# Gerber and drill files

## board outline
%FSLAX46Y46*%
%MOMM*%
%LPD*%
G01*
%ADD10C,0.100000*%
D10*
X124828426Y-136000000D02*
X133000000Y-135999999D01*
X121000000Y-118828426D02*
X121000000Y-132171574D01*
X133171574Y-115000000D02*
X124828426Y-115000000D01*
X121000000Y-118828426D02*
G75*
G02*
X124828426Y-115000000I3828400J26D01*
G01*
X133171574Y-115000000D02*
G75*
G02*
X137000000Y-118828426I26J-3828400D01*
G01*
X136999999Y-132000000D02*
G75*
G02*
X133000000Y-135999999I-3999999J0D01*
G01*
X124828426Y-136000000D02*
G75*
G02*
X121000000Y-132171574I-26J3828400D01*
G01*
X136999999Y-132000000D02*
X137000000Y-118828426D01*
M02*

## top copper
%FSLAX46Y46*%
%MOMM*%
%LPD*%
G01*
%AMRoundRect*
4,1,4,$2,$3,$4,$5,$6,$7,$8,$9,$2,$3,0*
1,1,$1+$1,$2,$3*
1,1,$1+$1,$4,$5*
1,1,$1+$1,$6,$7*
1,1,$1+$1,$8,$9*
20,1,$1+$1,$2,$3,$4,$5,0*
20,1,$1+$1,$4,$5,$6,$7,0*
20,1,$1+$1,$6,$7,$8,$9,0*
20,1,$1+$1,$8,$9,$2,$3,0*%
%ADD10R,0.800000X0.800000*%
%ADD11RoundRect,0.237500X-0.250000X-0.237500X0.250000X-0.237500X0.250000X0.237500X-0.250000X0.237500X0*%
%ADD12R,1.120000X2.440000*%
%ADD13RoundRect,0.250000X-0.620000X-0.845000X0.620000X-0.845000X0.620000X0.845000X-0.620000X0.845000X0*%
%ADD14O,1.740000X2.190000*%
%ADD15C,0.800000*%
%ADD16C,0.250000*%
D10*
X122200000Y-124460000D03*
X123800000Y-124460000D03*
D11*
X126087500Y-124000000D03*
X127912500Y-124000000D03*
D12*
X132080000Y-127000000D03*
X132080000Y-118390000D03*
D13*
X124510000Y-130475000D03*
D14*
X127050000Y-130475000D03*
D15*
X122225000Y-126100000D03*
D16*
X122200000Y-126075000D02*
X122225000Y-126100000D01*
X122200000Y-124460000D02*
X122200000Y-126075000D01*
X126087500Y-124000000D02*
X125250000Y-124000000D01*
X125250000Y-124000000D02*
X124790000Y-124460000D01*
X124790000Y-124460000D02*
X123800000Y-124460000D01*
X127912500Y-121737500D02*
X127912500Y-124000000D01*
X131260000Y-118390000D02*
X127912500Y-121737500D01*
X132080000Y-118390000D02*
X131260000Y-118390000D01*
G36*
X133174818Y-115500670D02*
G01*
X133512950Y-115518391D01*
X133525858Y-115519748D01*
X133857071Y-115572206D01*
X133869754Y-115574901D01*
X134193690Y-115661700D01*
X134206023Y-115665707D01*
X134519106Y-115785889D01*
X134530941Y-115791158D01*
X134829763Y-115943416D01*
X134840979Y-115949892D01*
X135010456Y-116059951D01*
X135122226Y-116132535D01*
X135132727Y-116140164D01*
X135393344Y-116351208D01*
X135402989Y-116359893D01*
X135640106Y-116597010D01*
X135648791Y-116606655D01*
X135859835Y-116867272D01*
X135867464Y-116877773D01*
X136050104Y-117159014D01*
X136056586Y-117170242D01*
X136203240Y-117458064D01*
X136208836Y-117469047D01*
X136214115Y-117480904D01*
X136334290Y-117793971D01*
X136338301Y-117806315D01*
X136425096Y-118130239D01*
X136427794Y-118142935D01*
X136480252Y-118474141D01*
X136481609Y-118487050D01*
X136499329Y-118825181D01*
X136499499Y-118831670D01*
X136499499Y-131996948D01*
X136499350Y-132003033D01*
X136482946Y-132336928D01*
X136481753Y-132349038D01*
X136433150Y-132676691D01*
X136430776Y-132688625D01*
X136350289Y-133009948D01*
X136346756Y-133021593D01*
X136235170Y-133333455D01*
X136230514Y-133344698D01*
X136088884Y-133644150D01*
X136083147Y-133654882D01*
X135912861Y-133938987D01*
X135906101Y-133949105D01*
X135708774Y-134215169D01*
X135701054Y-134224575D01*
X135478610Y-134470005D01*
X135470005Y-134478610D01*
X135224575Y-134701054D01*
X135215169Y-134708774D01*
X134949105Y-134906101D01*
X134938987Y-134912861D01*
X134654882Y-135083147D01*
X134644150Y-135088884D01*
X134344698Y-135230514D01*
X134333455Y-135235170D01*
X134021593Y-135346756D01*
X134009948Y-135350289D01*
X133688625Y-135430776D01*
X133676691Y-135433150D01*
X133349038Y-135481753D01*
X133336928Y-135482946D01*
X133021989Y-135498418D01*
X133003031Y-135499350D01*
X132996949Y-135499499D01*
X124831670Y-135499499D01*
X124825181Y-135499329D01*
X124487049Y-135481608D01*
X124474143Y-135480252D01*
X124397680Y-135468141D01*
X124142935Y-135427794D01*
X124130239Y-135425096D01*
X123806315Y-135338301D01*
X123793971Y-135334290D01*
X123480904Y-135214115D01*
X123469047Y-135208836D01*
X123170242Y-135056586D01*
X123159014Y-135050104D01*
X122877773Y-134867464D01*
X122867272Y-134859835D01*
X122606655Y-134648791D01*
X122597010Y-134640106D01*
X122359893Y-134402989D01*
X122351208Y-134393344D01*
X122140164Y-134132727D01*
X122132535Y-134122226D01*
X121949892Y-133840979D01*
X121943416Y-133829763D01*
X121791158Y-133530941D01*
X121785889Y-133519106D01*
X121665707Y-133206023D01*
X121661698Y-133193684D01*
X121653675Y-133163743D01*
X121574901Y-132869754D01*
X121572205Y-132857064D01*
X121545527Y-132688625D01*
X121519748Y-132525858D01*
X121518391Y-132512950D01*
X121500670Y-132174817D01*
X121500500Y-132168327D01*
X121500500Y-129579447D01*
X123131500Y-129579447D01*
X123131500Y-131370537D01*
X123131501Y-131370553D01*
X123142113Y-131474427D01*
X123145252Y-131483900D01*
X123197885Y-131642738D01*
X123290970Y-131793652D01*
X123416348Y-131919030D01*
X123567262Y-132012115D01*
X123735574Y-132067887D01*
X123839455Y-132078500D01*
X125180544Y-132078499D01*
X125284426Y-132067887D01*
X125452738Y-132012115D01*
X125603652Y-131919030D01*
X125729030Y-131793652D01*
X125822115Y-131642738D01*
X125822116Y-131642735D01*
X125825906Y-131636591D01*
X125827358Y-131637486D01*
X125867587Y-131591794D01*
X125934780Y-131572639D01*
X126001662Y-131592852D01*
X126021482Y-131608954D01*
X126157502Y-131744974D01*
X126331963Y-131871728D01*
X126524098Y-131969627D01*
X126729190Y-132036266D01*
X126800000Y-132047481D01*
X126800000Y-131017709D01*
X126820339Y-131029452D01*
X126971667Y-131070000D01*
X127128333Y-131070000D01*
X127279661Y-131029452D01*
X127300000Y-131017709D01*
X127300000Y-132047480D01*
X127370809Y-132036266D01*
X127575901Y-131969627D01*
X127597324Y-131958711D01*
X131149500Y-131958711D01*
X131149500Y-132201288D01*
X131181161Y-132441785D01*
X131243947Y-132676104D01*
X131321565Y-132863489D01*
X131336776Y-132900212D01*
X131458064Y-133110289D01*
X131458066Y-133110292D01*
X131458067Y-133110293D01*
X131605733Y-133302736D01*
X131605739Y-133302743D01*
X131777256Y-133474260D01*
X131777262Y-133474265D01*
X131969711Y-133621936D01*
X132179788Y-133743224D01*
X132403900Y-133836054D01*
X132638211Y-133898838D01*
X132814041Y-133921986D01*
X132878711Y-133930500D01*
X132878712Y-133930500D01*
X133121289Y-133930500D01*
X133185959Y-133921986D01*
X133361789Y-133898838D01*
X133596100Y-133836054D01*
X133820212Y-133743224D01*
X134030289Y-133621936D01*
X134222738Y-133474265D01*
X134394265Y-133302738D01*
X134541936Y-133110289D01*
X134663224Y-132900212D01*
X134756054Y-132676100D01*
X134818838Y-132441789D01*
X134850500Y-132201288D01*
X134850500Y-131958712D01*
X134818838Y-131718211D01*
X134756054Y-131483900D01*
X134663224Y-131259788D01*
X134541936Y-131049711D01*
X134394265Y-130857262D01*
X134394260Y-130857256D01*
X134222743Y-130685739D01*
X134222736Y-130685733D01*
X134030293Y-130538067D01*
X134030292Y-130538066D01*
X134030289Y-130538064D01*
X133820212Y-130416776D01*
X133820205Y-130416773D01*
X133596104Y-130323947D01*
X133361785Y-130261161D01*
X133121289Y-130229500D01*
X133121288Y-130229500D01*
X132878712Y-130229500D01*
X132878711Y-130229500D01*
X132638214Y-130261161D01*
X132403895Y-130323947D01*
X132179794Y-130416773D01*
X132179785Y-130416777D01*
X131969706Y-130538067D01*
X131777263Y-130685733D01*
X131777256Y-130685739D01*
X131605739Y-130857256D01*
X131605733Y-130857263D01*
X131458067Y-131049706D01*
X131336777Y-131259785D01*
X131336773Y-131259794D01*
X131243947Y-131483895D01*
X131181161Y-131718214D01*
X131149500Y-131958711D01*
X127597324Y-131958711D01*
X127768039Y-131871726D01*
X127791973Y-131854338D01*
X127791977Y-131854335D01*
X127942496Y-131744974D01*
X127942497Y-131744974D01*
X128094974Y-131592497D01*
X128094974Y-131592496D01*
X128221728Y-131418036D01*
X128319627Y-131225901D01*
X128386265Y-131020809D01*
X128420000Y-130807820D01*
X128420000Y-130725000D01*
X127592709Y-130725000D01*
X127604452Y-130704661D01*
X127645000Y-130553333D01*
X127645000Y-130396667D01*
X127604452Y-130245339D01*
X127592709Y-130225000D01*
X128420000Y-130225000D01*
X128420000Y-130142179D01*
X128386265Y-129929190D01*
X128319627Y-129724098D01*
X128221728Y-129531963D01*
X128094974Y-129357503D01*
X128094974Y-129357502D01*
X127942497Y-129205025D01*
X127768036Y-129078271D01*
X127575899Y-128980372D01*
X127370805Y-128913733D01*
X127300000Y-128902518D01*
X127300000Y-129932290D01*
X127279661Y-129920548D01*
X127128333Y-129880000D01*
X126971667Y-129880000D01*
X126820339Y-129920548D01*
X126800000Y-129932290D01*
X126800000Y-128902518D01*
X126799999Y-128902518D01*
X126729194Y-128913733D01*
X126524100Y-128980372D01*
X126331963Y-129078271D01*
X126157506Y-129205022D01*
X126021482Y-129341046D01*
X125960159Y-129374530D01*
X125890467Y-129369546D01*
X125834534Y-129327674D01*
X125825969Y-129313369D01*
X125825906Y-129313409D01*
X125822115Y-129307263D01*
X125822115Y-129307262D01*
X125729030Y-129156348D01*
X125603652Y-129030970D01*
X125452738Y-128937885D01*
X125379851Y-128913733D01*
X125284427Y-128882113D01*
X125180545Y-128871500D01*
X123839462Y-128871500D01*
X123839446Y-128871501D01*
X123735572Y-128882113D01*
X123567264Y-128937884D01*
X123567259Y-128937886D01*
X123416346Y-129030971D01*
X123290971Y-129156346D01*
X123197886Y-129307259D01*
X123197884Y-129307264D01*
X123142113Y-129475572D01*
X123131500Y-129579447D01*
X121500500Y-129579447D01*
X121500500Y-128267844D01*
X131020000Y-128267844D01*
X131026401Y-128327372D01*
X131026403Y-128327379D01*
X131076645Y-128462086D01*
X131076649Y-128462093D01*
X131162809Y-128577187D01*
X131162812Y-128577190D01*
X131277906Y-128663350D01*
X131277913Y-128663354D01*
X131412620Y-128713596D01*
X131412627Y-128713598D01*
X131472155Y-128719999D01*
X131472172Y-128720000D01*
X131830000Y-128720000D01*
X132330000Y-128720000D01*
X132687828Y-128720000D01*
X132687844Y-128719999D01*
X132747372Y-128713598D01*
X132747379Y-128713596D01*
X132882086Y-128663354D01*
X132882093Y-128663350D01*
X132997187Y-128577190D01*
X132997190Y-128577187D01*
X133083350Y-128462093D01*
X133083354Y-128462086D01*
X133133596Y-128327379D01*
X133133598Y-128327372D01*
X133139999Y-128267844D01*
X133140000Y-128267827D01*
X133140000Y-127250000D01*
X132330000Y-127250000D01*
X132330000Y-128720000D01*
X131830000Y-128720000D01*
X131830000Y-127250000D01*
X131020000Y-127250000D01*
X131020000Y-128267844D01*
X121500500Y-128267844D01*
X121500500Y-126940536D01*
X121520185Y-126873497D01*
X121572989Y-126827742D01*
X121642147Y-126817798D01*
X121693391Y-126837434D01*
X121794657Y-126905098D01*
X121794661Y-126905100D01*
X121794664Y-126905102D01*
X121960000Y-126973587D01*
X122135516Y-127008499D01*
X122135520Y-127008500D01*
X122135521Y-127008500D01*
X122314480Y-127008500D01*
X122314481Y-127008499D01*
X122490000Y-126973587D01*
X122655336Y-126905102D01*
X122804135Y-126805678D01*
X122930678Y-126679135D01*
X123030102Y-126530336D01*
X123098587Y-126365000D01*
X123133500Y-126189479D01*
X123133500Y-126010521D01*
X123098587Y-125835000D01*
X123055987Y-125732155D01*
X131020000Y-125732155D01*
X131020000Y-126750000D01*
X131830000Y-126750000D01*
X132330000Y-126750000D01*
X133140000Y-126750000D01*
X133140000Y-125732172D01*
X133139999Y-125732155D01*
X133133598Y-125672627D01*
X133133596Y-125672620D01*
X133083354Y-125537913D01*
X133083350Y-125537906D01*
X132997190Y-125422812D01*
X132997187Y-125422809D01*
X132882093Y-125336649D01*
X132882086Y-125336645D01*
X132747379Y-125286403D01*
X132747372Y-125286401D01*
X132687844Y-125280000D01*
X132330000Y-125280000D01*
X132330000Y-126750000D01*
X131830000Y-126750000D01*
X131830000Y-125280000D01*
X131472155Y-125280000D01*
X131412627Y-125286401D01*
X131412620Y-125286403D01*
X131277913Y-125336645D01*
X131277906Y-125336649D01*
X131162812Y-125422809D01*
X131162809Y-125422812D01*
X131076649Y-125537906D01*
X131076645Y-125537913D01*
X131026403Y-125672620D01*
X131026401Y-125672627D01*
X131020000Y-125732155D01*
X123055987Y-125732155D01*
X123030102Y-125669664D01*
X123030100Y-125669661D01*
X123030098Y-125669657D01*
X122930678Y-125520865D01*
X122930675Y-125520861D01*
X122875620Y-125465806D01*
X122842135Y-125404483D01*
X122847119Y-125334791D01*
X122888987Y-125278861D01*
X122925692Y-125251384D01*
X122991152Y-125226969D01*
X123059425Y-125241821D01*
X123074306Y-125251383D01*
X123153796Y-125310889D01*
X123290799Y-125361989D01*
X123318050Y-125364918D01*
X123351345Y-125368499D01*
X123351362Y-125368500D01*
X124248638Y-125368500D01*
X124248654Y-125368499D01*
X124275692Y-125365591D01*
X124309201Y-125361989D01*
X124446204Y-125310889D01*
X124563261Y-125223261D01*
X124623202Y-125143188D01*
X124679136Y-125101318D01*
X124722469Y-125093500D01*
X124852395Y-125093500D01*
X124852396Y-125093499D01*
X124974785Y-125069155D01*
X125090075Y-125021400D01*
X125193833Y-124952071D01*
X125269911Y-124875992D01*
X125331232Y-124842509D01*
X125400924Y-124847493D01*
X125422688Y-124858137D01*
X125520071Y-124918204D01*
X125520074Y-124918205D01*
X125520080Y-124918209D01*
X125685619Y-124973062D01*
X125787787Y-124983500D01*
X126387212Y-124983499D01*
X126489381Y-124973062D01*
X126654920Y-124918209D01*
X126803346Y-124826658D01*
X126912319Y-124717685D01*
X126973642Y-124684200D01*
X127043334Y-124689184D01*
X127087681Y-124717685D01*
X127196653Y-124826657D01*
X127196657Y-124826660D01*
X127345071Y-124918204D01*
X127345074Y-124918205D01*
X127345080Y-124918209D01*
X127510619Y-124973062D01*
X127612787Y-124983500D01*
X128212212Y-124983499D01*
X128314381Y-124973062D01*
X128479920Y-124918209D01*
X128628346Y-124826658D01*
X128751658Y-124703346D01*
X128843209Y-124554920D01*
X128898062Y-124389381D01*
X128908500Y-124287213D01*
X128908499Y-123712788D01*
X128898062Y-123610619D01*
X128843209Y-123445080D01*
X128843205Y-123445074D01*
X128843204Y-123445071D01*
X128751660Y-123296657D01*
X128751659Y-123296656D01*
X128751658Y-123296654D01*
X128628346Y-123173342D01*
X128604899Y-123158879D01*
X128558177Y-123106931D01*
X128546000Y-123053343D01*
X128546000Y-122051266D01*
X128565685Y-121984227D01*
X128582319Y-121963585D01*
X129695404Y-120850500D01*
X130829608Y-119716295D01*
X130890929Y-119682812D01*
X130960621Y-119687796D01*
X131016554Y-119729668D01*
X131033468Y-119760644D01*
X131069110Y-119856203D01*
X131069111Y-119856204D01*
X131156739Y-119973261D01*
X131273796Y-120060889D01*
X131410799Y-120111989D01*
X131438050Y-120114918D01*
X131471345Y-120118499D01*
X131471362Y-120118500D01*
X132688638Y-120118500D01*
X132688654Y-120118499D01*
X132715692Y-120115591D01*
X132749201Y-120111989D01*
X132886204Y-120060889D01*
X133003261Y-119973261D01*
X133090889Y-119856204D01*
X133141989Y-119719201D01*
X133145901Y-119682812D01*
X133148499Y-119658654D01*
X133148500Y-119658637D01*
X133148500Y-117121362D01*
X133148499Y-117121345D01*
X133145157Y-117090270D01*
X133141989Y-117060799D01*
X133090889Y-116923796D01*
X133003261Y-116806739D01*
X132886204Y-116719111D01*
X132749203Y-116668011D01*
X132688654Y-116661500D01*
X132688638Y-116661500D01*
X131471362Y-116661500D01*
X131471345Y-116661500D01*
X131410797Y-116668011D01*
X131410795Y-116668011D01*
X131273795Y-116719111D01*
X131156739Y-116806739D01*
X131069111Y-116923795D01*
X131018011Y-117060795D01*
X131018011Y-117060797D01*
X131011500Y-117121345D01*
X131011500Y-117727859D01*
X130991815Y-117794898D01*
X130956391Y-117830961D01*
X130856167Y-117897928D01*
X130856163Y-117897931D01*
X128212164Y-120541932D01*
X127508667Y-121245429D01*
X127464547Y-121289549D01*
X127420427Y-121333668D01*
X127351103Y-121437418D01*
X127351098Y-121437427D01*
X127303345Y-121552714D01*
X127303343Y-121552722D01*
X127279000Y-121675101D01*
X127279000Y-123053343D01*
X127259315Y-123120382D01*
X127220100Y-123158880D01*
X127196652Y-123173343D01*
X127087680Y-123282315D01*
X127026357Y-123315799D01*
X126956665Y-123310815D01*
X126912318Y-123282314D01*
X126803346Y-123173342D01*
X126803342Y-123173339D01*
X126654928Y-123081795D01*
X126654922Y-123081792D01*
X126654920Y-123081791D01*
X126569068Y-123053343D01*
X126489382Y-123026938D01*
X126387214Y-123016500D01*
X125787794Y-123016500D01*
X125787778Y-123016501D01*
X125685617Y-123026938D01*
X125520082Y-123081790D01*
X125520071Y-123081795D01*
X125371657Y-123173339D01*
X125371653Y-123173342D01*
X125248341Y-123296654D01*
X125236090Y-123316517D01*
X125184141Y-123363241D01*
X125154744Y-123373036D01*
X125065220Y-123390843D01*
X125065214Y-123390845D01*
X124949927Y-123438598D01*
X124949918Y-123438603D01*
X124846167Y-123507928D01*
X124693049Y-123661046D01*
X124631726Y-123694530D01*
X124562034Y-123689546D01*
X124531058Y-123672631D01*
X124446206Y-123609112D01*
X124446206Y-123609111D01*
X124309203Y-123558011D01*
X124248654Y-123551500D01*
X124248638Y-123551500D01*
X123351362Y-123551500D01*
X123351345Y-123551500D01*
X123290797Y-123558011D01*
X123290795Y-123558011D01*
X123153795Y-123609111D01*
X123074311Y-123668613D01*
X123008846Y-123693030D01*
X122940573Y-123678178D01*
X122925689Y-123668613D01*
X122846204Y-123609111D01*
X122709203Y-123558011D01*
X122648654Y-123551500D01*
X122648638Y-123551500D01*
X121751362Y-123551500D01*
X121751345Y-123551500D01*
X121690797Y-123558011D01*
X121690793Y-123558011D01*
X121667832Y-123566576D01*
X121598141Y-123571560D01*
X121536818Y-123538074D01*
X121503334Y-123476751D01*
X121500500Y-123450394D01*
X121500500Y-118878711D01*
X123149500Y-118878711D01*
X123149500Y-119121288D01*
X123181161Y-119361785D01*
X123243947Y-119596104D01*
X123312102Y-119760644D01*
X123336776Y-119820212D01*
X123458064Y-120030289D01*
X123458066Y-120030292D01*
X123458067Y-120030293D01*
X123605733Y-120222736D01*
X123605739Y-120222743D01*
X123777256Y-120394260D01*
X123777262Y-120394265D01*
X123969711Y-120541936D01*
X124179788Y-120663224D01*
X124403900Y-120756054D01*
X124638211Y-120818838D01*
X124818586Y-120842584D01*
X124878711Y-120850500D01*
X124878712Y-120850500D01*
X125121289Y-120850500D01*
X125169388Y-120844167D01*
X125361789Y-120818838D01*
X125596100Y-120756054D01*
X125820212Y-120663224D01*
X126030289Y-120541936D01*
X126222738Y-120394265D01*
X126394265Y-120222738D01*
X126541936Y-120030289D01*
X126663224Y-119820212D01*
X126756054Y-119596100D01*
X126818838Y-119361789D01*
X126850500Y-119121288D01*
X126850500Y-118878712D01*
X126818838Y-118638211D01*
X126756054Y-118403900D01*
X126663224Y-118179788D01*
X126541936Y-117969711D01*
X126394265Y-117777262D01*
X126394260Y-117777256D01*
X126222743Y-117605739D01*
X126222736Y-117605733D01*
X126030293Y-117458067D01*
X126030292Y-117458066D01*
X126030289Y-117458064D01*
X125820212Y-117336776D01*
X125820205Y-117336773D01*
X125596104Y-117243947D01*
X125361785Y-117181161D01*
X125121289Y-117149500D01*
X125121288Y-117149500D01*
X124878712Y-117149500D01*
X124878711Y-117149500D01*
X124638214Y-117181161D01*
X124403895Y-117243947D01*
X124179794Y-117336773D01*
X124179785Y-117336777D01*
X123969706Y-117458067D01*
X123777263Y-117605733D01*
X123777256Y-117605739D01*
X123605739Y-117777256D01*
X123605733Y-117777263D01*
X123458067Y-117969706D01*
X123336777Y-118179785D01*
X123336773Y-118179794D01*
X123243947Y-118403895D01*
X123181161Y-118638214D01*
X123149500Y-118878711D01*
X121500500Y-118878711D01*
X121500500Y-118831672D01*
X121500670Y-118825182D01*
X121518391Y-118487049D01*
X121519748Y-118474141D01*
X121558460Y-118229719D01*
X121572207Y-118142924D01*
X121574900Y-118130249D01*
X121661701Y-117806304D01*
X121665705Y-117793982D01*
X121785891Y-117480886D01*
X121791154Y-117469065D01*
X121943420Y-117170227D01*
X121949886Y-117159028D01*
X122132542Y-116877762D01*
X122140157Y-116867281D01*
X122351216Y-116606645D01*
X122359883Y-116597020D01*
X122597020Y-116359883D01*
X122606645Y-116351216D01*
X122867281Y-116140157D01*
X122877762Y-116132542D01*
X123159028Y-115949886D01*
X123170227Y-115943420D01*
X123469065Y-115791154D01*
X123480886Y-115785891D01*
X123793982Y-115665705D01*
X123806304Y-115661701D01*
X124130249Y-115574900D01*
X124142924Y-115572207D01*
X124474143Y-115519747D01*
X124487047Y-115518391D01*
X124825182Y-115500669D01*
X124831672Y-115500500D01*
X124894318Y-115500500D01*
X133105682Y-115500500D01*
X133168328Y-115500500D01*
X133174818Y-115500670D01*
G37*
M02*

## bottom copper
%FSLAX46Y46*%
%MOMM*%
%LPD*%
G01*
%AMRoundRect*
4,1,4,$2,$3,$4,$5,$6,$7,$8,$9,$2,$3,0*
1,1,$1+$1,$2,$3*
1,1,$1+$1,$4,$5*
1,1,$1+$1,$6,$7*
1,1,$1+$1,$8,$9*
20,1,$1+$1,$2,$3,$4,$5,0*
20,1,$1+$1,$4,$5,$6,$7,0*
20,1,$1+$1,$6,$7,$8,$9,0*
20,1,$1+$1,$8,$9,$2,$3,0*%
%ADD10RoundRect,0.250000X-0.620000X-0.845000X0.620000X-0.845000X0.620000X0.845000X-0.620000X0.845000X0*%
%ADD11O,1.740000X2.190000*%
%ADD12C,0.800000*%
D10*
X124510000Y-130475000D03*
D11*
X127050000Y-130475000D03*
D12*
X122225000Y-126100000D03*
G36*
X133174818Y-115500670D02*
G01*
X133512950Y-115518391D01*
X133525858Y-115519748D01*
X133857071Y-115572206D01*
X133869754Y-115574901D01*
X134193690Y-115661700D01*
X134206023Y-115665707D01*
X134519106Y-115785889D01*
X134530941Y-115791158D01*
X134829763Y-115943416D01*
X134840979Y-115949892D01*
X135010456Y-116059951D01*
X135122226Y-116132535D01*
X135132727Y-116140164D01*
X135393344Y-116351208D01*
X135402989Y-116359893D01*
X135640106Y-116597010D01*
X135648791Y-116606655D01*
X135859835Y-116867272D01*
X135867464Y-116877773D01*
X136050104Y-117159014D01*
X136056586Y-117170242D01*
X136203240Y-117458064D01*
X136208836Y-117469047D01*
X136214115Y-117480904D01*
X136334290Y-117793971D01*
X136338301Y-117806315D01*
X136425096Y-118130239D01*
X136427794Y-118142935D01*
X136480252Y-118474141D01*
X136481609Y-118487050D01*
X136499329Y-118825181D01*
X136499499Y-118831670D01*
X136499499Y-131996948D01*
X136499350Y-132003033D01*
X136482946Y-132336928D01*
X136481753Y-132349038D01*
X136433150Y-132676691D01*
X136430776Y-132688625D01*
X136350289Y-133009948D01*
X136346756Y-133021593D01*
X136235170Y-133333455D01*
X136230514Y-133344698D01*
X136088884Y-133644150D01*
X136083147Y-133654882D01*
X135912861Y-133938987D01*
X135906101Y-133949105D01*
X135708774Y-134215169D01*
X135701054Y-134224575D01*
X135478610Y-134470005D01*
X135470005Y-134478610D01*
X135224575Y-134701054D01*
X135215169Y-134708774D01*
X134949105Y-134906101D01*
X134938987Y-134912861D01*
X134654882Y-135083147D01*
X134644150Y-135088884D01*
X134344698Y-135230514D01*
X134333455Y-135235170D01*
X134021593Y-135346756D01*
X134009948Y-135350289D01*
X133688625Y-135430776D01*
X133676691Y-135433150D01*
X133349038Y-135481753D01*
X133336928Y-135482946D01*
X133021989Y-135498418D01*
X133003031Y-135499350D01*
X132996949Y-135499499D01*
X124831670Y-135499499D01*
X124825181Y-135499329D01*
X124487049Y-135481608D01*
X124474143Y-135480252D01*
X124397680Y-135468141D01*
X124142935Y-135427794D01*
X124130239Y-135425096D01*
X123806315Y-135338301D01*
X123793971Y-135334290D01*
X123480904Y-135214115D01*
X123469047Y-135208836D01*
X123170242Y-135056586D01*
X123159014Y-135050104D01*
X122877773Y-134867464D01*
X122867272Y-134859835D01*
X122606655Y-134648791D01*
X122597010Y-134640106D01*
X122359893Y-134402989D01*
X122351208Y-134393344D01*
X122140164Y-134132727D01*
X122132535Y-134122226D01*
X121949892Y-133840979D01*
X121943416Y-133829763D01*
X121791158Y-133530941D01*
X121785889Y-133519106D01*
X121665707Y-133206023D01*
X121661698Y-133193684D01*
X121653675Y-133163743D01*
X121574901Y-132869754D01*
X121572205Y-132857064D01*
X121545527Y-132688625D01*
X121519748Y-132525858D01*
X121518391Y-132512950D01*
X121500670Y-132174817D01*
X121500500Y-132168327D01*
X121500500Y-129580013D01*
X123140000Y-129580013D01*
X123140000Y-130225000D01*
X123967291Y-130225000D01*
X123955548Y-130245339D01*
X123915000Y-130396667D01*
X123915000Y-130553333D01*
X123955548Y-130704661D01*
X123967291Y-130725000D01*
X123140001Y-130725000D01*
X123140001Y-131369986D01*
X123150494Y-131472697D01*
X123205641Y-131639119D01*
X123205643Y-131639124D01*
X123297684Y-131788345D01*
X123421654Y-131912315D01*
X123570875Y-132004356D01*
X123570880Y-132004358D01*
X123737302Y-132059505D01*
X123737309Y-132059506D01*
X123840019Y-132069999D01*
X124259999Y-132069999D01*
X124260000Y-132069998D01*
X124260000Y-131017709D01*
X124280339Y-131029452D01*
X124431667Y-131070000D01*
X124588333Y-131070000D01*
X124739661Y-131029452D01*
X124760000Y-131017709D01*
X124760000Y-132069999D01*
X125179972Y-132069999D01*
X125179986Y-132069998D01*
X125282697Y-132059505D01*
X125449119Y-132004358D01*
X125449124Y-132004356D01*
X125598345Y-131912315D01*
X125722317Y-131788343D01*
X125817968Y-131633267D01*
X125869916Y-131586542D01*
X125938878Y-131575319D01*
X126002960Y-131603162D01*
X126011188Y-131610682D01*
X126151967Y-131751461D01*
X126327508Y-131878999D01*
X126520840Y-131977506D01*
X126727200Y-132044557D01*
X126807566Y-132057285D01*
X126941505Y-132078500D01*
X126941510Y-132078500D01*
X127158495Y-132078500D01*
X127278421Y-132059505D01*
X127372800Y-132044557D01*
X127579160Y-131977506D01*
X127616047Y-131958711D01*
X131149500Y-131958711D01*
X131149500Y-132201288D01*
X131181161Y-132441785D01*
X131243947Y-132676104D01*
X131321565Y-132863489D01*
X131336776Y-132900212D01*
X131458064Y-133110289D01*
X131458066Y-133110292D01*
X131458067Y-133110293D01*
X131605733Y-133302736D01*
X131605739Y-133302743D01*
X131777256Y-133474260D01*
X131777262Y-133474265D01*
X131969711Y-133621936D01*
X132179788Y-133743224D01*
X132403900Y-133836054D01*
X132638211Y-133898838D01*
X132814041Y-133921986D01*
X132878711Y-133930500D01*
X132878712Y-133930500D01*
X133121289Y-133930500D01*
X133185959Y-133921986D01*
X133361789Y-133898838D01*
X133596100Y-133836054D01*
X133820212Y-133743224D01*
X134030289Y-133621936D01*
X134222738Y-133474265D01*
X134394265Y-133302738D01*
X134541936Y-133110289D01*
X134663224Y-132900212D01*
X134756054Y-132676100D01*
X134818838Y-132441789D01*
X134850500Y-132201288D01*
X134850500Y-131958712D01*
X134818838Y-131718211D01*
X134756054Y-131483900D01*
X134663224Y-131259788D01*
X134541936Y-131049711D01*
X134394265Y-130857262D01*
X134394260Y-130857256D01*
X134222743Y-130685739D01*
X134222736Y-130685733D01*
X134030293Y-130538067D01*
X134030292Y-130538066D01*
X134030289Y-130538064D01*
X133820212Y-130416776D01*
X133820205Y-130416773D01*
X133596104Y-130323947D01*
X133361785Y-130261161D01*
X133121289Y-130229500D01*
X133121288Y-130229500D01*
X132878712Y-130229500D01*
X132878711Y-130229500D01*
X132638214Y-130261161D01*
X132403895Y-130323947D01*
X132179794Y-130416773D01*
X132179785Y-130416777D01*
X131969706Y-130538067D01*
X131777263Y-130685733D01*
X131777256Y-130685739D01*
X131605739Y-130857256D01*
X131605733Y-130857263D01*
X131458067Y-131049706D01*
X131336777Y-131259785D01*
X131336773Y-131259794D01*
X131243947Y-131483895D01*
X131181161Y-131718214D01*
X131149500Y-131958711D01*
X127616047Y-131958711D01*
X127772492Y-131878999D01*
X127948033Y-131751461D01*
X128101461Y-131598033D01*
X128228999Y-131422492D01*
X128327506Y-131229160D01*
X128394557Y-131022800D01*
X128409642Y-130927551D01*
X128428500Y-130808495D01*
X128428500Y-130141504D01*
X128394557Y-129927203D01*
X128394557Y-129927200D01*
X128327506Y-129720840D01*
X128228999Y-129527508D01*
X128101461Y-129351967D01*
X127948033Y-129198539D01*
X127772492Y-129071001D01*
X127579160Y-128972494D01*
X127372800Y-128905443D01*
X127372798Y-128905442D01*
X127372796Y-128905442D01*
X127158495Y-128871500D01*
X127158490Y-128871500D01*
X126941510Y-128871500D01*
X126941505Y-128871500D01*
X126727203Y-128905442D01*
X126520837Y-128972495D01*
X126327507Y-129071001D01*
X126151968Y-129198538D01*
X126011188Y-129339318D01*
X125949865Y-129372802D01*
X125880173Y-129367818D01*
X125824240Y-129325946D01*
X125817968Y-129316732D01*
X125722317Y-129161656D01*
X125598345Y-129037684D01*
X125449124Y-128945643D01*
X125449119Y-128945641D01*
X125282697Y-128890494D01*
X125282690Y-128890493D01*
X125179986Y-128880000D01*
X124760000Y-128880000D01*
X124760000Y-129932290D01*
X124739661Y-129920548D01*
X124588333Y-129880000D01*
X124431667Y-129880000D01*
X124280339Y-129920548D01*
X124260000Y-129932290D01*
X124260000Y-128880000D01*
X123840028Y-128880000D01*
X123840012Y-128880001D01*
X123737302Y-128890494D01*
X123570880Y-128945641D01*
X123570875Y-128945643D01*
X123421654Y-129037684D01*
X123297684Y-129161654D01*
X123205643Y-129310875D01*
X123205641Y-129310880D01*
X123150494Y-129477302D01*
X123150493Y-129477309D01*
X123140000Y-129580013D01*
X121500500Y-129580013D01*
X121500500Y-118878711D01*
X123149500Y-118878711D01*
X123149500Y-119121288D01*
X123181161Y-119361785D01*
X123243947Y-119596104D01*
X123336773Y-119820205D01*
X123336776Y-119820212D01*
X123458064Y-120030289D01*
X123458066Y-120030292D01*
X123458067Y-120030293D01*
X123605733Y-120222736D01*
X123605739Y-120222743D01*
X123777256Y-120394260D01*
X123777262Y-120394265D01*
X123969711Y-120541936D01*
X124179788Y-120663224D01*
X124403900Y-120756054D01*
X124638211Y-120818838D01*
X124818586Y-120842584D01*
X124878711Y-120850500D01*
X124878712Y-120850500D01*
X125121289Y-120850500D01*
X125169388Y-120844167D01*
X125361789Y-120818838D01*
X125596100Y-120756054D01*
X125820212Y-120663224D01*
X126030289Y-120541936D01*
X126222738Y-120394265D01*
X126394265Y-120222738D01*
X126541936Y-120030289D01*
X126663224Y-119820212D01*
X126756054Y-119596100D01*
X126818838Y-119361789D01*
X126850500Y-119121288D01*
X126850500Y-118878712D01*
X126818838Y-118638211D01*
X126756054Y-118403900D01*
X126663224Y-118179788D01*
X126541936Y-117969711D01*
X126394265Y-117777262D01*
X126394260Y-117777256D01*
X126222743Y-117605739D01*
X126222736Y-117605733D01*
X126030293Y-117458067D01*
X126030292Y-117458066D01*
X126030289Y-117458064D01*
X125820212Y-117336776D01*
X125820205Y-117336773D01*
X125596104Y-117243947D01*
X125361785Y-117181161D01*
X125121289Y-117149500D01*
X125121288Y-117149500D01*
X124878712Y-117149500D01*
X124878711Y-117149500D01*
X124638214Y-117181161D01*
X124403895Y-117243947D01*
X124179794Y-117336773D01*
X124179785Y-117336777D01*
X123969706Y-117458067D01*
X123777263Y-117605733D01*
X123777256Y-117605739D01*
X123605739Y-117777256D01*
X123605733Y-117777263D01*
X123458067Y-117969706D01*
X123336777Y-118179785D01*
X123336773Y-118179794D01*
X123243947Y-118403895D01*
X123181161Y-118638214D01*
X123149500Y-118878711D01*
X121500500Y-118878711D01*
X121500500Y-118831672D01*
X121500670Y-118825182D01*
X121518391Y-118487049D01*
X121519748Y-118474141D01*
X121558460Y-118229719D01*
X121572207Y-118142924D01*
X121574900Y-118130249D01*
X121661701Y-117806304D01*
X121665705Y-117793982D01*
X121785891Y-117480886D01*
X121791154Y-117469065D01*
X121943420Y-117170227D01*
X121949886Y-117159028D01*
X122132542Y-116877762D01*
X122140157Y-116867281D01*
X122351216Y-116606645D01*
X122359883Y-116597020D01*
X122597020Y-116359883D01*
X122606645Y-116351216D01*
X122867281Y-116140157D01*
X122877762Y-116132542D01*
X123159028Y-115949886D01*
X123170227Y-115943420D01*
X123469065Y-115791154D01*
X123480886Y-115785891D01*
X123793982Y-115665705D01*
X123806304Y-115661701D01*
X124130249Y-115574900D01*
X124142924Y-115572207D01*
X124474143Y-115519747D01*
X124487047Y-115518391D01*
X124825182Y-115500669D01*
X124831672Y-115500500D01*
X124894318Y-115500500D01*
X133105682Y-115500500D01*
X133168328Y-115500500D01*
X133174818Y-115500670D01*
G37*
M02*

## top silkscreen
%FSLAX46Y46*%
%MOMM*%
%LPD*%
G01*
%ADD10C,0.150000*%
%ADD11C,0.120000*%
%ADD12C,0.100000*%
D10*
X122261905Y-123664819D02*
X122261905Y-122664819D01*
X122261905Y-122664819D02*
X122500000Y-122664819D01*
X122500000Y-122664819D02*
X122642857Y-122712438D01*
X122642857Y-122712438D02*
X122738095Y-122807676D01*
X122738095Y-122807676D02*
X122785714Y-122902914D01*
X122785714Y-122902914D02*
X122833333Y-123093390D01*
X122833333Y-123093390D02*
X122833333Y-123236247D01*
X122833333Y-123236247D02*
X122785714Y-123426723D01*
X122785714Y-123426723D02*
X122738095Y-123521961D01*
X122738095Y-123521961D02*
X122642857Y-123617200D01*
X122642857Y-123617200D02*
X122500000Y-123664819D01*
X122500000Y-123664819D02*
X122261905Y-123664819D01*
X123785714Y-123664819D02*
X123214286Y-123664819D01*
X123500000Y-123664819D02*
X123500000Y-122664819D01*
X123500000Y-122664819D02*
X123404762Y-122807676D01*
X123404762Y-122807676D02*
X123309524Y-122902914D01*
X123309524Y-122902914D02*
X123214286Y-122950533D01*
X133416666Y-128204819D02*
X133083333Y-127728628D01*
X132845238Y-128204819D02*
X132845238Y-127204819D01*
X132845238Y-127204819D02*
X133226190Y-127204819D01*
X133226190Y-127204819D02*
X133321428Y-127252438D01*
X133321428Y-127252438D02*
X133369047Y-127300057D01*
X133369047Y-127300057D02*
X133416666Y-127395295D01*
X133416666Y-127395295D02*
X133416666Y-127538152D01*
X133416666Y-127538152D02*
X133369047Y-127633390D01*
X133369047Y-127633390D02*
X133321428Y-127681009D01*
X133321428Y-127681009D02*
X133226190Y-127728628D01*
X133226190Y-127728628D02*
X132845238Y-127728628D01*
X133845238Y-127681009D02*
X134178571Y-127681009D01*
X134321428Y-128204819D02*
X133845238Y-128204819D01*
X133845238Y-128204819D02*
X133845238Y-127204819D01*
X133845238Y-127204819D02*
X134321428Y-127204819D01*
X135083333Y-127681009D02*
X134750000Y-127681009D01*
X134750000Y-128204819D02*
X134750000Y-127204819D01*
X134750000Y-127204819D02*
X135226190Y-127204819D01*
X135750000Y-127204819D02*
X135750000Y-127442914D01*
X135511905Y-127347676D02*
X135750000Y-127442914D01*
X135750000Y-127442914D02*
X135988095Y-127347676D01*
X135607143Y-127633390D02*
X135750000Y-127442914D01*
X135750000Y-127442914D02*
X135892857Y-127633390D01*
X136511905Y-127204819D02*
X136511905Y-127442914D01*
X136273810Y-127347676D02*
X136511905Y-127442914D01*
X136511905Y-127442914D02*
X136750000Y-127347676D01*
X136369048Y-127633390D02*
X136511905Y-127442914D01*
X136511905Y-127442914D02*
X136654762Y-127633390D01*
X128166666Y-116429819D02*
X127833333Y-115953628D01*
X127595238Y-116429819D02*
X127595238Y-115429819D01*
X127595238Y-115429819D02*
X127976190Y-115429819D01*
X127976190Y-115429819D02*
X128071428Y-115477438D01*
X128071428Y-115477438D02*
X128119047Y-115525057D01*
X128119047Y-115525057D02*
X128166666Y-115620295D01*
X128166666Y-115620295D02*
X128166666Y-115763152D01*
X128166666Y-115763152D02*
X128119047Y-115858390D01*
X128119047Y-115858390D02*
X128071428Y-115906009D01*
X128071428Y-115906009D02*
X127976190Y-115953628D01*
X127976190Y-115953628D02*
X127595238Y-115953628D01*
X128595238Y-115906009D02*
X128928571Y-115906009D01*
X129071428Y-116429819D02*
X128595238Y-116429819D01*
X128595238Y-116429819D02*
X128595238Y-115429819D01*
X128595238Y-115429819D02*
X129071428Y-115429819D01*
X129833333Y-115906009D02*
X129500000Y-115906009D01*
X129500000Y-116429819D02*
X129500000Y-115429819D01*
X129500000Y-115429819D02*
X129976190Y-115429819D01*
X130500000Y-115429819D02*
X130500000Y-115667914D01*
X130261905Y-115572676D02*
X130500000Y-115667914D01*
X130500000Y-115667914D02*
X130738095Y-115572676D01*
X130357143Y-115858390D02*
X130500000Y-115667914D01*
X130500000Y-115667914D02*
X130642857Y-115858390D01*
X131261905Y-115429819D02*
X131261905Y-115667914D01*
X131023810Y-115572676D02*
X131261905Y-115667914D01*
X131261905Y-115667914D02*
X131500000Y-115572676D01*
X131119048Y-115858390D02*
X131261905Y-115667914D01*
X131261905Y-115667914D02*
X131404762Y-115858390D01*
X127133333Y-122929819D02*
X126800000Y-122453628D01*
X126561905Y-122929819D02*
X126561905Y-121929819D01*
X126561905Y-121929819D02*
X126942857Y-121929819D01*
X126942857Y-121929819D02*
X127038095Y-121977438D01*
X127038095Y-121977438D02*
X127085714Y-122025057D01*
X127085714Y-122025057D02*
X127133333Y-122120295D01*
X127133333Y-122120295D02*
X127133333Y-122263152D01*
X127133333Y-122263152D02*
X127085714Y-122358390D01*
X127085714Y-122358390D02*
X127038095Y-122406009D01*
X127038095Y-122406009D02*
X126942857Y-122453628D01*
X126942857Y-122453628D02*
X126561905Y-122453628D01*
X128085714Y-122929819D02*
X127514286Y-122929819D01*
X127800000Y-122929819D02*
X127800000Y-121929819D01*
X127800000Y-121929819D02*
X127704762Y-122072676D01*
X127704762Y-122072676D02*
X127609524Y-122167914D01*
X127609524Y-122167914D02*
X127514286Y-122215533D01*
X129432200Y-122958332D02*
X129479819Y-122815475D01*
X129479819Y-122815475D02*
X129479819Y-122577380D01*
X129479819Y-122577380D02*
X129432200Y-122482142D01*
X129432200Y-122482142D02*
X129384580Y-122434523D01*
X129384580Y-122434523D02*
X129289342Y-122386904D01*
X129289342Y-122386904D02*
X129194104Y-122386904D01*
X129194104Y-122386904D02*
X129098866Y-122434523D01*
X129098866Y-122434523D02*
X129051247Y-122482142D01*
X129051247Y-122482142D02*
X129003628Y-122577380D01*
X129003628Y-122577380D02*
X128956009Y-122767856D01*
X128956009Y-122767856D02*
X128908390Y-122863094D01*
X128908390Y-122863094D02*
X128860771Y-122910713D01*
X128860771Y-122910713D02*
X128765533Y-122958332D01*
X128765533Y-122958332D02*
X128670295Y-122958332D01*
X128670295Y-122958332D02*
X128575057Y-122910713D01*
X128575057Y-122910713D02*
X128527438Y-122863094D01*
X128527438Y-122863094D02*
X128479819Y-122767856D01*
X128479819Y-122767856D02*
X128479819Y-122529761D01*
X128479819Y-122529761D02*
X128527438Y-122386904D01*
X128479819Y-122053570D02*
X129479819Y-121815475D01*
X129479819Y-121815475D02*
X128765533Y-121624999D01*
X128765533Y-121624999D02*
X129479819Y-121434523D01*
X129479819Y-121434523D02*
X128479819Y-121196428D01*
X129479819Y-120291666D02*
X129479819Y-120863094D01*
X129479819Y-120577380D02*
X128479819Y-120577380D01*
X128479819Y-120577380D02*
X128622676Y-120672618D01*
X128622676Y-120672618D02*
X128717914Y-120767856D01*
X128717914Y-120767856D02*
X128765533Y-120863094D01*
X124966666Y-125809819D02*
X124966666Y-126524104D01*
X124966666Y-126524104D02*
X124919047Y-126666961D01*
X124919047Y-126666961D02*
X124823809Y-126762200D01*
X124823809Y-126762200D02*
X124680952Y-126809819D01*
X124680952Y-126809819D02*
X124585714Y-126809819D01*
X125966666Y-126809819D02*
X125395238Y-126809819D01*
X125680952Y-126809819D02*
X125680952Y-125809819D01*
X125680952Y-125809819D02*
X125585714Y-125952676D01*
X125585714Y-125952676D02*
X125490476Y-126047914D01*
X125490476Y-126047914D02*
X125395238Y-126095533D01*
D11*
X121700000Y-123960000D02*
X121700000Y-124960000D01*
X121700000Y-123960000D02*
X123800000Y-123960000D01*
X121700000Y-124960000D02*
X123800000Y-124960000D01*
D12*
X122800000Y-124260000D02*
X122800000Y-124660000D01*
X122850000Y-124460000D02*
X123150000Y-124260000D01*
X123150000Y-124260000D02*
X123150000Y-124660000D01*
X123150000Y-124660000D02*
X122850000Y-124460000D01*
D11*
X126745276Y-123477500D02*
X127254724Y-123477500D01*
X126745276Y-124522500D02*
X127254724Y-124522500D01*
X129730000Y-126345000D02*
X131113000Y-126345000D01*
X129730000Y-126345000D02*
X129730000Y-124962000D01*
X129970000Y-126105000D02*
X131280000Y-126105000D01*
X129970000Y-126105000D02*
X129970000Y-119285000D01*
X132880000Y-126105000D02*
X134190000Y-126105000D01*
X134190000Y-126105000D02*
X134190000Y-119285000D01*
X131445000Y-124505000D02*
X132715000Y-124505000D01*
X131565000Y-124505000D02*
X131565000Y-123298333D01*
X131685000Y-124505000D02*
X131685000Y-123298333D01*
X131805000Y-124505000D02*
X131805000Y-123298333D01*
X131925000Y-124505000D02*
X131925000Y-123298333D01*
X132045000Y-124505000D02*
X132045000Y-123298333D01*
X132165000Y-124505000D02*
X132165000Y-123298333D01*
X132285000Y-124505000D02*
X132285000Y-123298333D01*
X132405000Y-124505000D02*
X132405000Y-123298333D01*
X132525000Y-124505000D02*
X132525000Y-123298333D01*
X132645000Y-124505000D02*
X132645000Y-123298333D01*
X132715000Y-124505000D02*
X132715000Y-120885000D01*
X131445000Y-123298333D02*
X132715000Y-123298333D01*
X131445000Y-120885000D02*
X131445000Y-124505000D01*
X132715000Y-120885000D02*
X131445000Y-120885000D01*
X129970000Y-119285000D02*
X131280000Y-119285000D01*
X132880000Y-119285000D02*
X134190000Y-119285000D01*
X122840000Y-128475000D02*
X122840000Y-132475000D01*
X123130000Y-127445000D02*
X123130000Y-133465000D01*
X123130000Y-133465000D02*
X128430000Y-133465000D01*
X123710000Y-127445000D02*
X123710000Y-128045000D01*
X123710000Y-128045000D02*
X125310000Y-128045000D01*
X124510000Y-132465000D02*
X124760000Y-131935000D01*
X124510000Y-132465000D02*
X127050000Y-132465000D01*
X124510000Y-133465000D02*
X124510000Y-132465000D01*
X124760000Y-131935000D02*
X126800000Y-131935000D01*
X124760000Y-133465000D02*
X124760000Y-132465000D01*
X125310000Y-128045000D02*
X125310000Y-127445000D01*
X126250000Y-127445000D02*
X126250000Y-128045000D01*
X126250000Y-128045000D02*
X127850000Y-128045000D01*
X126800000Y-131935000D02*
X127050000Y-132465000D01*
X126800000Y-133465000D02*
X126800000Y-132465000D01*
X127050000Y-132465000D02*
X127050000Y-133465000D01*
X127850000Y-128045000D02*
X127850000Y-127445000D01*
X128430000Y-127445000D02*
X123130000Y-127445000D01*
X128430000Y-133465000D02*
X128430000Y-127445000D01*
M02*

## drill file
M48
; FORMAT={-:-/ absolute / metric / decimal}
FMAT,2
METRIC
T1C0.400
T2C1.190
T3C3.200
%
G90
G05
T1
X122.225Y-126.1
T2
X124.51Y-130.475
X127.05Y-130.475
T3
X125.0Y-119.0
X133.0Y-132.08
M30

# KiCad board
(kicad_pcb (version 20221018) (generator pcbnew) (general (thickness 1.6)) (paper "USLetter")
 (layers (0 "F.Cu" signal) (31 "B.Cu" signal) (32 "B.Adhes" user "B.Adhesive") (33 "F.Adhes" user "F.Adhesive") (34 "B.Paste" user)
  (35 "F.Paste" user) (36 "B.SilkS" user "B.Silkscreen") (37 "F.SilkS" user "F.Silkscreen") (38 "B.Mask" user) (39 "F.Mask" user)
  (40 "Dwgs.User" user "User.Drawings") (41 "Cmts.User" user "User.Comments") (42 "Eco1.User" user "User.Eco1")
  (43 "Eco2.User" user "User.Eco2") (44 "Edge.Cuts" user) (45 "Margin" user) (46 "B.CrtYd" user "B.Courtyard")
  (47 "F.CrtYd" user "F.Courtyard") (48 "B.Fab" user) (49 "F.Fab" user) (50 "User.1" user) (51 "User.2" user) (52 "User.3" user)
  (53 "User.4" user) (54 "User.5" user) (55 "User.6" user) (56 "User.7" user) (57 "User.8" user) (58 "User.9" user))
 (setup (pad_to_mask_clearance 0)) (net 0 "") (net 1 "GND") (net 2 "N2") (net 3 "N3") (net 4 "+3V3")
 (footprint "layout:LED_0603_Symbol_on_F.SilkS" (layer "F.Cu") (at 123 124.46)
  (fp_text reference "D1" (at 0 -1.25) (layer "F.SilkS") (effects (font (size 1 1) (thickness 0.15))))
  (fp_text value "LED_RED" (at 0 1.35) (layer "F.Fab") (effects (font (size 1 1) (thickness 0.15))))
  (fp_line (start -1.3 -0.5) (end -1.3 0.5) (stroke (width 0.12) (type solid)) (layer "F.SilkS"))
  (fp_line (start -1.3 -0.5) (end 0.8 -0.5) (stroke (width 0.12) (type solid)) (layer "F.SilkS"))
  (fp_line (start -1.3 0.5) (end 0.8 0.5) (stroke (width 0.12) (type solid)) (layer "F.SilkS"))
  (fp_line (start -0.2 -0.2) (end -0.2 0.2) (stroke (width 0.1) (type solid)) (layer "F.SilkS"))
  (fp_line (start -0.15 0) (end 0.15 -0.2) (stroke (width 0.1) (type solid)) (layer "F.SilkS"))
  (fp_line (start 0.15 -0.2) (end 0.15 0.2) (stroke (width 0.1) (type solid)) (layer "F.SilkS"))
  (fp_line (start 0.15 0.2) (end -0.15 0) (stroke (width 0.1) (type solid)) (layer "F.SilkS"))
  (pad "1" smd rect (at -0.8 0 180) (size 0.8 0.8) (layers "F.Cu" "F.Paste" "F.Mask") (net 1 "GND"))
  (pad "2" smd rect (at 0.8 0 180) (size 0.8 0.8) (layers "F.Cu" "F.Paste" "F.Mask") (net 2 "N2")))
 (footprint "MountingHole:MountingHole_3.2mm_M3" (layer "F.Cu") (at 133 132.08)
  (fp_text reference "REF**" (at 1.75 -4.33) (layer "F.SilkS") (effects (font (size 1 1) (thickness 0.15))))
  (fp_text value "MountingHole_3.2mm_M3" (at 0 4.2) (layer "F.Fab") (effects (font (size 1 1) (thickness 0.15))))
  (pad "" np_thru_hole circle (at 0 0) (size 3.2 3.2) (drill 3.2) (layers "*.Cu" "*.Mask")))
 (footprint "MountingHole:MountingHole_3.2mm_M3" (layer "F.Cu") (at 125 119)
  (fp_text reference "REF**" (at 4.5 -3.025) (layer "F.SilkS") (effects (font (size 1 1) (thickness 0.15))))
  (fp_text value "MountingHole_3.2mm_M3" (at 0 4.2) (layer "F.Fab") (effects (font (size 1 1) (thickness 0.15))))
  (pad "" np_thru_hole circle (at 0 0) (size 3.2 3.2) (drill 3.2) (layers "F&B.Cu" "*.Mask")))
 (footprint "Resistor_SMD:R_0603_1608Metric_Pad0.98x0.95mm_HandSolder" (layer "F.Cu") (at 127 124)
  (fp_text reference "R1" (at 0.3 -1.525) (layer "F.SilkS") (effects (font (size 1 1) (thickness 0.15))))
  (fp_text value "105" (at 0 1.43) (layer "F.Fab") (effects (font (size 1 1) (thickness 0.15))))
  (fp_line (start -0.254724 -0.5225) (end 0.254724 -0.5225) (stroke (width 0.12) (type solid)) (layer "F.SilkS"))
  (fp_line (start -0.254724 0.5225) (end 0.254724 0.5225) (stroke (width 0.12) (type solid)) (layer "F.SilkS"))
  (pad "1" smd roundrect (at -0.9125 0) (size 0.975 0.95) (layers "F.Cu" "F.Paste" "F.Mask") (roundrect_rratio 0.25) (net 2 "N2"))
  (pad "2" smd roundrect (at 0.9125 0) (size 0.975 0.95) (layers "F.Cu" "F.Paste" "F.Mask") (roundrect_rratio 0.25) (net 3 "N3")))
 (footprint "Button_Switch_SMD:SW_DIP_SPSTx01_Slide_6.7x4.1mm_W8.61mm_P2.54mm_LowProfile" (layer "F.Cu") (at 132.08 122.695 90)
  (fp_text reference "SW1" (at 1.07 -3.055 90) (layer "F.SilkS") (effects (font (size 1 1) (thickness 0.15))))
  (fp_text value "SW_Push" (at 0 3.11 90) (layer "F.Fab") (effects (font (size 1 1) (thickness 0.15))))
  (fp_line (start -3.65 -2.35) (end -3.65 -0.967) (stroke (width 0.12) (type solid)) (layer "F.SilkS"))
  (fp_line (start -3.65 -2.35) (end -2.267 -2.35) (stroke (width 0.12) (type solid)) (layer "F.SilkS"))
  (fp_line (start -3.41 -2.11) (end -3.41 -0.8) (stroke (width 0.12) (type solid)) (layer "F.SilkS"))
  (fp_line (start -3.41 -2.11) (end 3.41 -2.11) (stroke (width 0.12) (type solid)) (layer "F.SilkS"))
  (fp_line (start -3.41 0.8) (end -3.41 2.11) (stroke (width 0.12) (type solid)) (layer "F.SilkS"))
  (fp_line (start -3.41 2.11) (end 3.41 2.11) (stroke (width 0.12) (type solid)) (layer "F.SilkS"))
  (fp_line (start -1.81 -0.635) (end -1.81 0.635) (stroke (width 0.12) (type solid)) (layer "F.SilkS"))
  (fp_line (start -1.81 -0.515) (end -0.603333 -0.515) (stroke (width 0.12) (type solid)) (layer "F.SilkS"))
  (fp_line (start -1.81 -0.395) (end -0.603333 -0.395) (stroke (width 0.12) (type solid)) (layer "F.SilkS"))
  (fp_line (start -1.81 -0.275) (end -0.603333 -0.275) (stroke (width 0.12) (type solid)) (layer "F.SilkS"))
  (fp_line (start -1.81 -0.155) (end -0.603333 -0.155) (stroke (width 0.12) (type solid)) (layer "F.SilkS"))
  (fp_line (start -1.81 -0.035) (end -0.603333 -0.035) (stroke (width 0.12) (type solid)) (layer "F.SilkS"))
  (fp_line (start -1.81 0.085) (end -0.603333 0.085) (stroke (width 0.12) (type solid)) (layer "F.SilkS"))
  (fp_line (start -1.81 0.205) (end -0.603333 0.205) (stroke (width 0.12) (type solid)) (layer "F.SilkS"))
  (fp_line (start -1.81 0.325) (end -0.603333 0.325) (stroke (width 0.12) (type solid)) (layer "F.SilkS"))
  (fp_line (start -1.81 0.445) (end -0.603333 0.445) (stroke (width 0.12) (type solid)) (layer "F.SilkS"))
  (fp_line (start -1.81 0.565) (end -0.603333 0.565) (stroke (width 0.12) (type solid)) (layer "F.SilkS"))
  (fp_line (start -1.81 0.635) (end 1.81 0.635) (stroke (width 0.12) (type solid)) (layer "F.SilkS"))
  (fp_line (start -0.603333 -0.635) (end -0.603333 0.635) (stroke (width 0.12) (type solid)) (layer "F.SilkS"))
  (fp_line (start 1.81 -0.635) (end -1.81 -0.635) (stroke (width 0.12) (type solid)) (layer "F.SilkS"))
  (fp_line (start 1.81 0.635) (end 1.81 -0.635) (stroke (width 0.12) (type solid)) (layer "F.SilkS"))
  (fp_line (start 3.41 -2.11) (end 3.41 -0.8) (stroke (width 0.12) (type solid)) (layer "F.SilkS"))
  (fp_line (start 3.41 0.8) (end 3.41 2.11) (stroke (width 0.12) (type solid)) (layer "F.SilkS"))
  (pad "1" smd rect (at -4.305 0 90) (size 2.44 1.12) (layers "F.Cu" "F.Paste" "F.Mask") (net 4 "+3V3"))
  (pad "2" smd rect (at 4.305 0 90) (size 2.44 1.12) (layers "F.Cu" "F.Paste" "F.Mask") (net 3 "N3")))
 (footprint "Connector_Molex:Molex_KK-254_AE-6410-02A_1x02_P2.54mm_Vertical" (layer "F.Cu") (at 124.51 130.475)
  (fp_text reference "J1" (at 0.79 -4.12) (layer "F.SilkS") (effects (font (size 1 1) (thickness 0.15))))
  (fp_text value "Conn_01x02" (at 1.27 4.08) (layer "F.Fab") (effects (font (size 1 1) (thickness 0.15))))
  (fp_line (start -1.67 -2) (end -1.67 2) (stroke (width 0.12) (type solid)) (layer "F.SilkS"))
  (fp_line (start -1.38 -3.03) (end -1.38 2.99) (stroke (width 0.12) (type solid)) (layer "F.SilkS"))
  (fp_line (start -1.38 2.99) (end 3.92 2.99) (stroke (width 0.12) (type solid)) (layer "F.SilkS"))
  (fp_line (start -0.8 -3.03) (end -0.8 -2.43) (stroke (width 0.12) (type solid)) (layer "F.SilkS"))
  (fp_line (start -0.8 -2.43) (end 0.8 -2.43) (stroke (width 0.12) (type solid)) (layer "F.SilkS"))
  (fp_line (start 0 1.99) (end 0.25 1.46) (stroke (width 0.12) (type solid)) (layer "F.SilkS"))
  (fp_line (start 0 1.99) (end 2.54 1.99) (stroke (width 0.12) (type solid)) (layer "F.SilkS"))
  (fp_line (start 0 2.99) (end 0 1.99) (stroke (width 0.12) (type solid)) (layer "F.SilkS"))
  (fp_line (start 0.25 1.46) (end 2.29 1.46) (stroke (width 0.12) (type solid)) (layer "F.SilkS"))
  (fp_line (start 0.25 2.99) (end 0.25 1.99) (stroke (width 0.12) (type solid)) (layer "F.SilkS"))
  (fp_line (start 0.8 -2.43) (end 0.8 -3.03) (stroke (width 0.12) (type solid)) (layer "F.SilkS"))
  (fp_line (start 1.74 -3.03) (end 1.74 -2.43) (stroke (width 0.12) (type solid)) (layer "F.SilkS"))
  (fp_line (start 1.74 -2.43) (end 3.34 -2.43) (stroke (width 0.12) (type solid)) (layer "F.SilkS"))
  (fp_line (start 2.29 1.46) (end 2.54 1.99) (stroke (width 0.12) (type solid)) (layer "F.SilkS"))
  (fp_line (start 2.29 2.99) (end 2.29 1.99) (stroke (width 0.12) (type solid)) (layer "F.SilkS"))
  (fp_line (start 2.54 1.99) (end 2.54 2.99) (stroke (width 0.12) (type solid)) (layer "F.SilkS"))
  (fp_line (start 3.34 -2.43) (end 3.34 -3.03) (stroke (width 0.12) (type solid)) (layer "F.SilkS"))
  (fp_line (start 3.92 -3.03) (end -1.38 -3.03) (stroke (width 0.12) (type solid)) (layer "F.SilkS"))
  (fp_line (start 3.92 2.99) (end 3.92 -3.03) (stroke (width 0.12) (type solid)) (layer "F.SilkS"))
  (pad "1" thru_hole roundrect (at 0 0) (size 1.74 2.19) (drill 1.19) (layers "*.Cu" "*.Mask") (roundrect_rratio 0.143678) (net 1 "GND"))
  (pad "2" thru_hole oval (at 2.54 0) (size 1.74 2.19) (drill 1.19) (layers "*.Cu" "*.Mask") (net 4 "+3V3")))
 (gr_line (start 124.828426 136) (end 133 135.999999) (stroke (width 0.1) (type default)) (layer "Edge.Cuts"))
 (gr_line (start 121 118.828426) (end 121 132.171574) (stroke (width 0.1) (type default)) (layer "Edge.Cuts"))
 (gr_line (start 133.171574 115) (end 124.828426 115) (stroke (width 0.1) (type default)) (layer "Edge.Cuts"))
 (gr_arc (start 121 118.828426) (mid 122.12132 116.12132) (end 124.828426 115) (stroke (width 0.1) (type default)) (layer "Edge.Cuts"))
 (gr_arc (start 133.171574 115) (mid 135.87868 116.12132) (end 137 118.828426) (stroke (width 0.1) (type default)) (layer "Edge.Cuts"))
 (gr_arc (start 136.999999 132) (mid 135.828426 134.828426) (end 133 135.999999) (stroke (width 0.1) (type default)) (layer "Edge.Cuts"))
 (gr_arc (start 124.828426 136) (mid 122.12132 134.87868) (end 121 132.171574) (stroke (width 0.1) (type default)) (layer "Edge.Cuts"))
 (gr_line (start 136.999999 132) (end 137 118.828426) (stroke (width 0.1) (type default)) (layer "Edge.Cuts"))
 (segment (start 122.2 126.075) (end 122.225 126.1) (width 0.25) (layer "F.Cu") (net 1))
 (segment (start 122.2 124.46) (end 122.2 126.075) (width 0.25) (layer "F.Cu") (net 1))
 (via (at 122.225 126.1) (size 0.8) (drill 0.4) (layers "F.Cu" "B.Cu") (free) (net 1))
 (segment (start 126.0875 124) (end 125.25 124) (width 0.25) (layer "F.Cu") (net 2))
 (segment (start 125.25 124) (end 124.79 124.46) (width 0.25) (layer "F.Cu") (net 2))
 (segment (start 124.79 124.46) (end 123.8 124.46) (width 0.25) (layer "F.Cu") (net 2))
 (segment (start 127.9125 121.7375) (end 127.9125 124) (width 0.25) (layer "F.Cu") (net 3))
 (segment (start 131.26 118.39) (end 127.9125 121.7375) (width 0.25) (layer "F.Cu") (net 3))
 (segment (start 132.08 118.39) (end 131.26 118.39) (width 0.25) (layer "F.Cu") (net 3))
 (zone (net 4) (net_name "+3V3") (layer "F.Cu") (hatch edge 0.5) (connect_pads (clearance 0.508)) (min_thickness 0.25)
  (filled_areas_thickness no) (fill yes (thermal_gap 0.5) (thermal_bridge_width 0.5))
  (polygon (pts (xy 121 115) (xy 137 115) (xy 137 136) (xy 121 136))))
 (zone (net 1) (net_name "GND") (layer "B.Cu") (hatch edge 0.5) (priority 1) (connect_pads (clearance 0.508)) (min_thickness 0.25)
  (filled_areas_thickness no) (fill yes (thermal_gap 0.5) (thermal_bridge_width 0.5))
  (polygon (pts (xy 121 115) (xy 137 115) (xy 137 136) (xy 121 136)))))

